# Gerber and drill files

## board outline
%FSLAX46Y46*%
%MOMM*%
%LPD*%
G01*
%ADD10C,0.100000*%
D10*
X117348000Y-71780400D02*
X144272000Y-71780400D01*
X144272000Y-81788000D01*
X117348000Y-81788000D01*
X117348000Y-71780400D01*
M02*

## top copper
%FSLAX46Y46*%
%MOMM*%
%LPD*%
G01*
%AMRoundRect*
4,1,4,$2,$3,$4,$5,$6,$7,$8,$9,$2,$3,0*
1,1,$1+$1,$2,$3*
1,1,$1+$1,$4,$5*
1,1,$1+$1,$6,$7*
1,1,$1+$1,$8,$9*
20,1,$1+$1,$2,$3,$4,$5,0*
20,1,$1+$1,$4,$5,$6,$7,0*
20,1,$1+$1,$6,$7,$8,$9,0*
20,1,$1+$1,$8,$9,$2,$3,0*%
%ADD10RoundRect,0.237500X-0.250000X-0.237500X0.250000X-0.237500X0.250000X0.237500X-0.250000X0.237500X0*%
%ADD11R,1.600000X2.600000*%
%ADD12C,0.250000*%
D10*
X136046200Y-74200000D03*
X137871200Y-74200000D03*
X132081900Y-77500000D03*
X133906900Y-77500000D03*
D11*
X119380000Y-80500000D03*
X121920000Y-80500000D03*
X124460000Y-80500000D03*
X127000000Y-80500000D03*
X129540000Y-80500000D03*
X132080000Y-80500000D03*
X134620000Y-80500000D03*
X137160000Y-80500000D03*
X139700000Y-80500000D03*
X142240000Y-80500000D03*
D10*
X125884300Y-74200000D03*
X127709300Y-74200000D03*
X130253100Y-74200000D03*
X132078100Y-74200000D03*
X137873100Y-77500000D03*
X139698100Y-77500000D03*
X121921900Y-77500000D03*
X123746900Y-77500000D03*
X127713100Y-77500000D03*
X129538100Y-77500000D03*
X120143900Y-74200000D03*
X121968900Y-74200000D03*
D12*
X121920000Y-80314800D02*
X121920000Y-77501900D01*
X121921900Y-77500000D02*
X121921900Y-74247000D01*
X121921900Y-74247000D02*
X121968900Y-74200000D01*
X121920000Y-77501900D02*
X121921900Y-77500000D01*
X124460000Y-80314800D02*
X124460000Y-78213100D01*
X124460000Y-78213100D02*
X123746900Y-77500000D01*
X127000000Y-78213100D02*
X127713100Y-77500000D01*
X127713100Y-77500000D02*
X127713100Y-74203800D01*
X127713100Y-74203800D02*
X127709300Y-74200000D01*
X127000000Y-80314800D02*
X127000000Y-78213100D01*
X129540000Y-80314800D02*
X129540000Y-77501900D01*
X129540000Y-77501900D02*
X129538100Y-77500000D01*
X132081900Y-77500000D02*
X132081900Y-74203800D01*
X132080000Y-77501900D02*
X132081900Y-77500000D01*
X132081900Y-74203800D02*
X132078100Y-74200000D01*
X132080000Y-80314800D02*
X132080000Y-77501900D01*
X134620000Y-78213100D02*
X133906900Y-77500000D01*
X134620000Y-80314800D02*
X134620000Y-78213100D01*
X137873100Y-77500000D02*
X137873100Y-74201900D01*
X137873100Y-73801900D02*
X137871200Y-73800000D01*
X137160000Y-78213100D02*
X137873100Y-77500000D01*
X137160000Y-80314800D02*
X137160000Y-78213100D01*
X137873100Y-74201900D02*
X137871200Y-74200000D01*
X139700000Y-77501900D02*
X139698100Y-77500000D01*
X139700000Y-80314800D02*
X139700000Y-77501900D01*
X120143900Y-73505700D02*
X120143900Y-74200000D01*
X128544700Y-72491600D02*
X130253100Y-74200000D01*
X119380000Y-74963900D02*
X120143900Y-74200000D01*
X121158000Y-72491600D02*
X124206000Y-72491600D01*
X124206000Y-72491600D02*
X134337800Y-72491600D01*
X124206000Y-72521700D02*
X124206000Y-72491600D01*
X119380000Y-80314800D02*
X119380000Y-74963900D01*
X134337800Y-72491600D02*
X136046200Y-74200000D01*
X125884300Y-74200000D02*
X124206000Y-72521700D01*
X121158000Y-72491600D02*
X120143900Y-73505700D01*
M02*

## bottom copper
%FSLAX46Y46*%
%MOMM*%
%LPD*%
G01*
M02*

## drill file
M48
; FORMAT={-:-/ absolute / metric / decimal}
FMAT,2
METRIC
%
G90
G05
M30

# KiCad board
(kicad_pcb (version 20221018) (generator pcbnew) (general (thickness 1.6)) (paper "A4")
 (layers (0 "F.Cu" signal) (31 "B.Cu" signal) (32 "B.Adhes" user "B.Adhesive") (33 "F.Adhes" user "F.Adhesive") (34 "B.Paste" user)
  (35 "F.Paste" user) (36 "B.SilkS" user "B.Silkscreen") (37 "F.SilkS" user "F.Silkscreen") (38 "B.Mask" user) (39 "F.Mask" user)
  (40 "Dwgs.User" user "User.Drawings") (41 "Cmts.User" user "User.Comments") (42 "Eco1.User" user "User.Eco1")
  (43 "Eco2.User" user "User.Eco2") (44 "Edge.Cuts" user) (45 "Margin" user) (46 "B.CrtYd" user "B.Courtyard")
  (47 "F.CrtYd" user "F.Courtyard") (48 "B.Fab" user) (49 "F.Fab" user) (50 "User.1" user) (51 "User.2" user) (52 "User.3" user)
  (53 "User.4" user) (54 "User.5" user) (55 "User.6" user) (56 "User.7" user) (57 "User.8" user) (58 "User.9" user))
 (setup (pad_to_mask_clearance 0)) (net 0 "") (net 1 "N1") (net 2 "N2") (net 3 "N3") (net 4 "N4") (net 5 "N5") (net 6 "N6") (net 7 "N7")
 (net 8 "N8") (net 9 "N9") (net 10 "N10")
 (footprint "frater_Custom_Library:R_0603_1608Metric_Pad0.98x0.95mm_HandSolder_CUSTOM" (layer "F.Cu") (at 136.9587 74.2)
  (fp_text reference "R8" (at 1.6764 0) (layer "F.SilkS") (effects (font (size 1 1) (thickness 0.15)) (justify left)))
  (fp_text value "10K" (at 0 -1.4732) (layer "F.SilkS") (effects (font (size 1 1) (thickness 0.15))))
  (pad "1" smd roundrect (at -0.9125 0) (size 0.975 0.95) (layers "F.Cu" "F.Paste" "F.Mask") (roundrect_rratio 0.25) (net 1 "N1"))
  (pad "2" smd roundrect (at 0.9125 0) (size 0.975 0.95) (layers "F.Cu" "F.Paste" "F.Mask") (roundrect_rratio 0.25) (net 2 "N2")))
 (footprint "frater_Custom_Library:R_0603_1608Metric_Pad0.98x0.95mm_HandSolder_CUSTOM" (layer "F.Cu") (at 132.9944 77.5)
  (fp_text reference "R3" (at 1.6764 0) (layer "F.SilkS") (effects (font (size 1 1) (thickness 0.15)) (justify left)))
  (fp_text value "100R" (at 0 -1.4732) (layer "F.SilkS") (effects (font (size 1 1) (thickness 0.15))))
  (pad "1" smd roundrect (at -0.9125 0) (size 0.975 0.95) (layers "F.Cu" "F.Paste" "F.Mask") (roundrect_rratio 0.25) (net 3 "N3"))
  (pad "2" smd roundrect (at 0.9125 0) (size 0.975 0.95) (layers "F.Cu" "F.Paste" "F.Mask") (roundrect_rratio 0.25) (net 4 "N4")))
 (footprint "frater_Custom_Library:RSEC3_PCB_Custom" (layer "F.Cu") (at 119.38 80.5)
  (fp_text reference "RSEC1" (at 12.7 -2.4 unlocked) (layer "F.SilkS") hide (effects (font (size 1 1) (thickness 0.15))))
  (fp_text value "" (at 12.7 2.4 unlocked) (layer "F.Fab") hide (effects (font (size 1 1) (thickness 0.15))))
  (pad "1" smd rect (at 0 0) (size 1.6 2.6) (layers "F.Cu" "F.Paste" "F.Mask") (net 1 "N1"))
  (pad "2" smd rect (at 2.54 0) (size 1.6 2.6) (layers "F.Cu" "F.Paste" "F.Mask") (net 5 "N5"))
  (pad "3" smd rect (at 5.08 0) (size 1.6 2.6) (layers "F.Cu" "F.Paste" "F.Mask") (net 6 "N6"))
  (pad "4" smd rect (at 7.62 0) (size 1.6 2.6) (layers "F.Cu" "F.Paste" "F.Mask") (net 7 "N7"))
  (pad "5" smd rect (at 10.16 0) (size 1.6 2.6) (layers "F.Cu" "F.Paste" "F.Mask") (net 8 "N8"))
  (pad "6" smd rect (at 12.7 0) (size 1.6 2.6) (layers "F.Cu" "F.Paste" "F.Mask") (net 3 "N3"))
  (pad "7" smd rect (at 15.24 0) (size 1.6 2.6) (layers "F.Cu" "F.Paste" "F.Mask") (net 4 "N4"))
  (pad "8" smd rect (at 17.78 0) (size 1.6 2.6) (layers "F.Cu" "F.Paste" "F.Mask") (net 2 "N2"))
  (pad "9" smd rect (at 20.32 0) (size 1.6 2.6) (layers "F.Cu" "F.Paste" "F.Mask") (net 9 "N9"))
  (pad "10" smd rect (at 22.86 0) (size 1.6 2.6) (layers "F.Cu" "F.Paste" "F.Mask") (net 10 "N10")))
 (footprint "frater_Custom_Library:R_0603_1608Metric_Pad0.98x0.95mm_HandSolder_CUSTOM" (layer "F.Cu") (at 126.7968 74.2)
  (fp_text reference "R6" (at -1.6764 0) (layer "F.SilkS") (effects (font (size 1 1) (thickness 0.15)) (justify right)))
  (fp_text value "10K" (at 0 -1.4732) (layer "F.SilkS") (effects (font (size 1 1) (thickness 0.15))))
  (pad "1" smd roundrect (at -0.9125 0) (size 0.975 0.95) (layers "F.Cu" "F.Paste" "F.Mask") (roundrect_rratio 0.25) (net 1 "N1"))
  (pad "2" smd roundrect (at 0.9125 0) (size 0.975 0.95) (layers "F.Cu" "F.Paste" "F.Mask") (roundrect_rratio 0.25) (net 7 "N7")))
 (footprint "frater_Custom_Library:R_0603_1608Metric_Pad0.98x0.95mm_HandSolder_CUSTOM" (layer "F.Cu") (at 131.1656 74.2)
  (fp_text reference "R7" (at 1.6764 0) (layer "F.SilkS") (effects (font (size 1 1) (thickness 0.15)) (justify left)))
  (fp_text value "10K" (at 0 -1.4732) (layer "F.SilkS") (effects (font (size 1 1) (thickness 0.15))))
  (pad "1" smd roundrect (at -0.9125 0) (size 0.975 0.95) (layers "F.Cu" "F.Paste" "F.Mask") (roundrect_rratio 0.25) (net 1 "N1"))
  (pad "2" smd roundrect (at 0.9125 0) (size 0.975 0.95) (layers "F.Cu" "F.Paste" "F.Mask") (roundrect_rratio 0.25) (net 3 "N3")))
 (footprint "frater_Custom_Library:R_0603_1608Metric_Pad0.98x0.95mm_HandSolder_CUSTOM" (layer "F.Cu") (at 138.7856 77.5)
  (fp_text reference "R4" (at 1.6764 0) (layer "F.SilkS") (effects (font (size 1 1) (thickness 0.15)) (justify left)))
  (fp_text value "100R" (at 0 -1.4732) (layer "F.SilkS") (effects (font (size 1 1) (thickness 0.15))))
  (pad "1" smd roundrect (at -0.9125 0) (size 0.975 0.95) (layers "F.Cu" "F.Paste" "F.Mask") (roundrect_rratio 0.25) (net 2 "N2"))
  (pad "2" smd roundrect (at 0.9125 0) (size 0.975 0.95) (layers "F.Cu" "F.Paste" "F.Mask") (roundrect_rratio 0.25) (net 9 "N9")))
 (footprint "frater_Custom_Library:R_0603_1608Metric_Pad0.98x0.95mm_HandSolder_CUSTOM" (layer "F.Cu") (at 122.8344 77.5)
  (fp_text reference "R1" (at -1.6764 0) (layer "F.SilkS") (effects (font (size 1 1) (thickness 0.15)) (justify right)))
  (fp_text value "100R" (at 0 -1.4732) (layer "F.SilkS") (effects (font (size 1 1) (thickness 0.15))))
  (pad "1" smd roundrect (at -0.9125 0) (size 0.975 0.95) (layers "F.Cu" "F.Paste" "F.Mask") (roundrect_rratio 0.25) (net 5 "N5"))
  (pad "2" smd roundrect (at 0.9125 0) (size 0.975 0.95) (layers "F.Cu" "F.Paste" "F.Mask") (roundrect_rratio 0.25) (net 6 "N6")))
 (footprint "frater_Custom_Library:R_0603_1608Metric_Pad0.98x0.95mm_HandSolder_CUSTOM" (layer "F.Cu") (at 128.6256 77.5)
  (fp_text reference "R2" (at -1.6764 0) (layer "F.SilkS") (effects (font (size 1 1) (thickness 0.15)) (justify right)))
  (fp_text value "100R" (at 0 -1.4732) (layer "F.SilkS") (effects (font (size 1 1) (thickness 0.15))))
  (pad "1" smd roundrect (at -0.9125 0) (size 0.975 0.95) (layers "F.Cu" "F.Paste" "F.Mask") (roundrect_rratio 0.25) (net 7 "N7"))
  (pad "2" smd roundrect (at 0.9125 0) (size 0.975 0.95) (layers "F.Cu" "F.Paste" "F.Mask") (roundrect_rratio 0.25) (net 8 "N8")))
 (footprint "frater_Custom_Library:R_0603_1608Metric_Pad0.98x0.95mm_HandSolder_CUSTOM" (layer "F.Cu") (at 121.0564 74.2)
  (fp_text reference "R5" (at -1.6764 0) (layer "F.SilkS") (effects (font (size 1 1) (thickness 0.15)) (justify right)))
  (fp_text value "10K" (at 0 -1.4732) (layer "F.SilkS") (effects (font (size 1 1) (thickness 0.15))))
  (pad "1" smd roundrect (at -0.9125 0) (size 0.975 0.95) (layers "F.Cu" "F.Paste" "F.Mask") (roundrect_rratio 0.25) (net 1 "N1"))
  (pad "2" smd roundrect (at 0.9125 0) (size 0.975 0.95) (layers "F.Cu" "F.Paste" "F.Mask") (roundrect_rratio 0.25) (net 5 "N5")))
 (gr_rect (start 117.348 71.7804) (end 144.272 81.788) (stroke (width 0.1) (type default)) (fill none) (layer "Edge.Cuts"))
 (segment (start 121.92 80.3148) (end 121.92 77.5019) (width 0.25) (layer "F.Cu") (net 5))
 (segment (start 121.9219 77.5) (end 121.9219 74.247) (width 0.25) (layer "F.Cu") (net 5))
 (segment (start 121.9219 74.247) (end 121.9689 74.2) (width 0.25) (layer "F.Cu") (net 5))
 (segment (start 121.92 77.5019) (end 121.9219 77.5) (width 0.25) (layer "F.Cu") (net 5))
 (segment (start 124.46 80.3148) (end 124.46 78.2131) (width 0.25) (layer "F.Cu") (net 6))
 (segment (start 124.46 78.2131) (end 123.7469 77.5) (width 0.25) (layer "F.Cu") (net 6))
 (segment (start 127 78.2131) (end 127.7131 77.5) (width 0.25) (layer "F.Cu") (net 7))
 (segment (start 127.7131 77.5) (end 127.7131 74.2038) (width 0.25) (layer "F.Cu") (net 7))
 (segment (start 127.7131 74.2038) (end 127.7093 74.2) (width 0.25) (layer "F.Cu") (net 7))
 (segment (start 127 80.3148) (end 127 78.2131) (width 0.25) (layer "F.Cu") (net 7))
 (segment (start 129.54 80.3148) (end 129.54 77.5019) (width 0.25) (layer "F.Cu") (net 8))
 (segment (start 129.54 77.5019) (end 129.5381 77.5) (width 0.25) (layer "F.Cu") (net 8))
 (segment (start 132.0819 77.5) (end 132.0819 74.2038) (width 0.25) (layer "F.Cu") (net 3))
 (segment (start 132.08 77.5019) (end 132.0819 77.5) (width 0.25) (layer "F.Cu") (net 3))
 (segment (start 132.0819 74.2038) (end 132.0781 74.2) (width 0.25) (layer "F.Cu") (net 3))
 (segment (start 132.08 80.3148) (end 132.08 77.5019) (width 0.25) (layer "F.Cu") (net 3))
 (segment (start 134.62 78.2131) (end 133.9069 77.5) (width 0.25) (layer "F.Cu") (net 4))
 (segment (start 134.62 80.3148) (end 134.62 78.2131) (width 0.25) (layer "F.Cu") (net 4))
 (segment (start 137.8731 77.5) (end 137.8731 74.2019) (width 0.25) (layer "F.Cu") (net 2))
 (segment (start 137.8731 73.8019) (end 137.8712 73.8) (width 0.25) (layer "F.Cu") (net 2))
 (segment (start 137.16 78.2131) (end 137.8731 77.5) (width 0.25) (layer "F.Cu") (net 2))
 (segment (start 137.16 80.3148) (end 137.16 78.2131) (width 0.25) (layer "F.Cu") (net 2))
 (segment (start 137.8731 74.2019) (end 137.8712 74.2) (width 0.25) (layer "F.Cu") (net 2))
 (segment (start 139.7 77.5019) (end 139.6981 77.5) (width 0.25) (layer "F.Cu") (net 9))
 (segment (start 139.7 80.3148) (end 139.7 77.5019) (width 0.25) (layer "F.Cu") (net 9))
 (segment (start 120.1439 73.5057) (end 120.1439 74.2) (width 0.25) (layer "F.Cu") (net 1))
 (segment (start 128.5447 72.4916) (end 130.2531 74.2) (width 0.25) (layer "F.Cu") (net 1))
 (segment (start 119.38 74.9639) (end 120.1439 74.2) (width 0.25) (layer "F.Cu") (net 1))
 (segment (start 121.158 72.4916) (end 124.206 72.4916) (width 0.25) (layer "F.Cu") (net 1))
 (segment (start 124.206 72.4916) (end 134.3378 72.4916) (width 0.25) (layer "F.Cu") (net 1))
 (segment (start 124.206 72.5217) (end 124.206 72.4916) (width 0.25) (layer "F.Cu") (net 1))
 (segment (start 119.38 80.3148) (end 119.38 74.9639) (width 0.25) (layer "F.Cu") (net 1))
 (segment (start 134.3378 72.4916) (end 136.0462 74.2) (width 0.25) (layer "F.Cu") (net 1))
 (segment (start 125.8843 74.2) (end 124.206 72.5217) (width 0.25) (layer "F.Cu") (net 1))
 (segment (start 121.158 72.4916) (end 120.1439 73.5057) (width 0.25) (layer "F.Cu") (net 1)))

